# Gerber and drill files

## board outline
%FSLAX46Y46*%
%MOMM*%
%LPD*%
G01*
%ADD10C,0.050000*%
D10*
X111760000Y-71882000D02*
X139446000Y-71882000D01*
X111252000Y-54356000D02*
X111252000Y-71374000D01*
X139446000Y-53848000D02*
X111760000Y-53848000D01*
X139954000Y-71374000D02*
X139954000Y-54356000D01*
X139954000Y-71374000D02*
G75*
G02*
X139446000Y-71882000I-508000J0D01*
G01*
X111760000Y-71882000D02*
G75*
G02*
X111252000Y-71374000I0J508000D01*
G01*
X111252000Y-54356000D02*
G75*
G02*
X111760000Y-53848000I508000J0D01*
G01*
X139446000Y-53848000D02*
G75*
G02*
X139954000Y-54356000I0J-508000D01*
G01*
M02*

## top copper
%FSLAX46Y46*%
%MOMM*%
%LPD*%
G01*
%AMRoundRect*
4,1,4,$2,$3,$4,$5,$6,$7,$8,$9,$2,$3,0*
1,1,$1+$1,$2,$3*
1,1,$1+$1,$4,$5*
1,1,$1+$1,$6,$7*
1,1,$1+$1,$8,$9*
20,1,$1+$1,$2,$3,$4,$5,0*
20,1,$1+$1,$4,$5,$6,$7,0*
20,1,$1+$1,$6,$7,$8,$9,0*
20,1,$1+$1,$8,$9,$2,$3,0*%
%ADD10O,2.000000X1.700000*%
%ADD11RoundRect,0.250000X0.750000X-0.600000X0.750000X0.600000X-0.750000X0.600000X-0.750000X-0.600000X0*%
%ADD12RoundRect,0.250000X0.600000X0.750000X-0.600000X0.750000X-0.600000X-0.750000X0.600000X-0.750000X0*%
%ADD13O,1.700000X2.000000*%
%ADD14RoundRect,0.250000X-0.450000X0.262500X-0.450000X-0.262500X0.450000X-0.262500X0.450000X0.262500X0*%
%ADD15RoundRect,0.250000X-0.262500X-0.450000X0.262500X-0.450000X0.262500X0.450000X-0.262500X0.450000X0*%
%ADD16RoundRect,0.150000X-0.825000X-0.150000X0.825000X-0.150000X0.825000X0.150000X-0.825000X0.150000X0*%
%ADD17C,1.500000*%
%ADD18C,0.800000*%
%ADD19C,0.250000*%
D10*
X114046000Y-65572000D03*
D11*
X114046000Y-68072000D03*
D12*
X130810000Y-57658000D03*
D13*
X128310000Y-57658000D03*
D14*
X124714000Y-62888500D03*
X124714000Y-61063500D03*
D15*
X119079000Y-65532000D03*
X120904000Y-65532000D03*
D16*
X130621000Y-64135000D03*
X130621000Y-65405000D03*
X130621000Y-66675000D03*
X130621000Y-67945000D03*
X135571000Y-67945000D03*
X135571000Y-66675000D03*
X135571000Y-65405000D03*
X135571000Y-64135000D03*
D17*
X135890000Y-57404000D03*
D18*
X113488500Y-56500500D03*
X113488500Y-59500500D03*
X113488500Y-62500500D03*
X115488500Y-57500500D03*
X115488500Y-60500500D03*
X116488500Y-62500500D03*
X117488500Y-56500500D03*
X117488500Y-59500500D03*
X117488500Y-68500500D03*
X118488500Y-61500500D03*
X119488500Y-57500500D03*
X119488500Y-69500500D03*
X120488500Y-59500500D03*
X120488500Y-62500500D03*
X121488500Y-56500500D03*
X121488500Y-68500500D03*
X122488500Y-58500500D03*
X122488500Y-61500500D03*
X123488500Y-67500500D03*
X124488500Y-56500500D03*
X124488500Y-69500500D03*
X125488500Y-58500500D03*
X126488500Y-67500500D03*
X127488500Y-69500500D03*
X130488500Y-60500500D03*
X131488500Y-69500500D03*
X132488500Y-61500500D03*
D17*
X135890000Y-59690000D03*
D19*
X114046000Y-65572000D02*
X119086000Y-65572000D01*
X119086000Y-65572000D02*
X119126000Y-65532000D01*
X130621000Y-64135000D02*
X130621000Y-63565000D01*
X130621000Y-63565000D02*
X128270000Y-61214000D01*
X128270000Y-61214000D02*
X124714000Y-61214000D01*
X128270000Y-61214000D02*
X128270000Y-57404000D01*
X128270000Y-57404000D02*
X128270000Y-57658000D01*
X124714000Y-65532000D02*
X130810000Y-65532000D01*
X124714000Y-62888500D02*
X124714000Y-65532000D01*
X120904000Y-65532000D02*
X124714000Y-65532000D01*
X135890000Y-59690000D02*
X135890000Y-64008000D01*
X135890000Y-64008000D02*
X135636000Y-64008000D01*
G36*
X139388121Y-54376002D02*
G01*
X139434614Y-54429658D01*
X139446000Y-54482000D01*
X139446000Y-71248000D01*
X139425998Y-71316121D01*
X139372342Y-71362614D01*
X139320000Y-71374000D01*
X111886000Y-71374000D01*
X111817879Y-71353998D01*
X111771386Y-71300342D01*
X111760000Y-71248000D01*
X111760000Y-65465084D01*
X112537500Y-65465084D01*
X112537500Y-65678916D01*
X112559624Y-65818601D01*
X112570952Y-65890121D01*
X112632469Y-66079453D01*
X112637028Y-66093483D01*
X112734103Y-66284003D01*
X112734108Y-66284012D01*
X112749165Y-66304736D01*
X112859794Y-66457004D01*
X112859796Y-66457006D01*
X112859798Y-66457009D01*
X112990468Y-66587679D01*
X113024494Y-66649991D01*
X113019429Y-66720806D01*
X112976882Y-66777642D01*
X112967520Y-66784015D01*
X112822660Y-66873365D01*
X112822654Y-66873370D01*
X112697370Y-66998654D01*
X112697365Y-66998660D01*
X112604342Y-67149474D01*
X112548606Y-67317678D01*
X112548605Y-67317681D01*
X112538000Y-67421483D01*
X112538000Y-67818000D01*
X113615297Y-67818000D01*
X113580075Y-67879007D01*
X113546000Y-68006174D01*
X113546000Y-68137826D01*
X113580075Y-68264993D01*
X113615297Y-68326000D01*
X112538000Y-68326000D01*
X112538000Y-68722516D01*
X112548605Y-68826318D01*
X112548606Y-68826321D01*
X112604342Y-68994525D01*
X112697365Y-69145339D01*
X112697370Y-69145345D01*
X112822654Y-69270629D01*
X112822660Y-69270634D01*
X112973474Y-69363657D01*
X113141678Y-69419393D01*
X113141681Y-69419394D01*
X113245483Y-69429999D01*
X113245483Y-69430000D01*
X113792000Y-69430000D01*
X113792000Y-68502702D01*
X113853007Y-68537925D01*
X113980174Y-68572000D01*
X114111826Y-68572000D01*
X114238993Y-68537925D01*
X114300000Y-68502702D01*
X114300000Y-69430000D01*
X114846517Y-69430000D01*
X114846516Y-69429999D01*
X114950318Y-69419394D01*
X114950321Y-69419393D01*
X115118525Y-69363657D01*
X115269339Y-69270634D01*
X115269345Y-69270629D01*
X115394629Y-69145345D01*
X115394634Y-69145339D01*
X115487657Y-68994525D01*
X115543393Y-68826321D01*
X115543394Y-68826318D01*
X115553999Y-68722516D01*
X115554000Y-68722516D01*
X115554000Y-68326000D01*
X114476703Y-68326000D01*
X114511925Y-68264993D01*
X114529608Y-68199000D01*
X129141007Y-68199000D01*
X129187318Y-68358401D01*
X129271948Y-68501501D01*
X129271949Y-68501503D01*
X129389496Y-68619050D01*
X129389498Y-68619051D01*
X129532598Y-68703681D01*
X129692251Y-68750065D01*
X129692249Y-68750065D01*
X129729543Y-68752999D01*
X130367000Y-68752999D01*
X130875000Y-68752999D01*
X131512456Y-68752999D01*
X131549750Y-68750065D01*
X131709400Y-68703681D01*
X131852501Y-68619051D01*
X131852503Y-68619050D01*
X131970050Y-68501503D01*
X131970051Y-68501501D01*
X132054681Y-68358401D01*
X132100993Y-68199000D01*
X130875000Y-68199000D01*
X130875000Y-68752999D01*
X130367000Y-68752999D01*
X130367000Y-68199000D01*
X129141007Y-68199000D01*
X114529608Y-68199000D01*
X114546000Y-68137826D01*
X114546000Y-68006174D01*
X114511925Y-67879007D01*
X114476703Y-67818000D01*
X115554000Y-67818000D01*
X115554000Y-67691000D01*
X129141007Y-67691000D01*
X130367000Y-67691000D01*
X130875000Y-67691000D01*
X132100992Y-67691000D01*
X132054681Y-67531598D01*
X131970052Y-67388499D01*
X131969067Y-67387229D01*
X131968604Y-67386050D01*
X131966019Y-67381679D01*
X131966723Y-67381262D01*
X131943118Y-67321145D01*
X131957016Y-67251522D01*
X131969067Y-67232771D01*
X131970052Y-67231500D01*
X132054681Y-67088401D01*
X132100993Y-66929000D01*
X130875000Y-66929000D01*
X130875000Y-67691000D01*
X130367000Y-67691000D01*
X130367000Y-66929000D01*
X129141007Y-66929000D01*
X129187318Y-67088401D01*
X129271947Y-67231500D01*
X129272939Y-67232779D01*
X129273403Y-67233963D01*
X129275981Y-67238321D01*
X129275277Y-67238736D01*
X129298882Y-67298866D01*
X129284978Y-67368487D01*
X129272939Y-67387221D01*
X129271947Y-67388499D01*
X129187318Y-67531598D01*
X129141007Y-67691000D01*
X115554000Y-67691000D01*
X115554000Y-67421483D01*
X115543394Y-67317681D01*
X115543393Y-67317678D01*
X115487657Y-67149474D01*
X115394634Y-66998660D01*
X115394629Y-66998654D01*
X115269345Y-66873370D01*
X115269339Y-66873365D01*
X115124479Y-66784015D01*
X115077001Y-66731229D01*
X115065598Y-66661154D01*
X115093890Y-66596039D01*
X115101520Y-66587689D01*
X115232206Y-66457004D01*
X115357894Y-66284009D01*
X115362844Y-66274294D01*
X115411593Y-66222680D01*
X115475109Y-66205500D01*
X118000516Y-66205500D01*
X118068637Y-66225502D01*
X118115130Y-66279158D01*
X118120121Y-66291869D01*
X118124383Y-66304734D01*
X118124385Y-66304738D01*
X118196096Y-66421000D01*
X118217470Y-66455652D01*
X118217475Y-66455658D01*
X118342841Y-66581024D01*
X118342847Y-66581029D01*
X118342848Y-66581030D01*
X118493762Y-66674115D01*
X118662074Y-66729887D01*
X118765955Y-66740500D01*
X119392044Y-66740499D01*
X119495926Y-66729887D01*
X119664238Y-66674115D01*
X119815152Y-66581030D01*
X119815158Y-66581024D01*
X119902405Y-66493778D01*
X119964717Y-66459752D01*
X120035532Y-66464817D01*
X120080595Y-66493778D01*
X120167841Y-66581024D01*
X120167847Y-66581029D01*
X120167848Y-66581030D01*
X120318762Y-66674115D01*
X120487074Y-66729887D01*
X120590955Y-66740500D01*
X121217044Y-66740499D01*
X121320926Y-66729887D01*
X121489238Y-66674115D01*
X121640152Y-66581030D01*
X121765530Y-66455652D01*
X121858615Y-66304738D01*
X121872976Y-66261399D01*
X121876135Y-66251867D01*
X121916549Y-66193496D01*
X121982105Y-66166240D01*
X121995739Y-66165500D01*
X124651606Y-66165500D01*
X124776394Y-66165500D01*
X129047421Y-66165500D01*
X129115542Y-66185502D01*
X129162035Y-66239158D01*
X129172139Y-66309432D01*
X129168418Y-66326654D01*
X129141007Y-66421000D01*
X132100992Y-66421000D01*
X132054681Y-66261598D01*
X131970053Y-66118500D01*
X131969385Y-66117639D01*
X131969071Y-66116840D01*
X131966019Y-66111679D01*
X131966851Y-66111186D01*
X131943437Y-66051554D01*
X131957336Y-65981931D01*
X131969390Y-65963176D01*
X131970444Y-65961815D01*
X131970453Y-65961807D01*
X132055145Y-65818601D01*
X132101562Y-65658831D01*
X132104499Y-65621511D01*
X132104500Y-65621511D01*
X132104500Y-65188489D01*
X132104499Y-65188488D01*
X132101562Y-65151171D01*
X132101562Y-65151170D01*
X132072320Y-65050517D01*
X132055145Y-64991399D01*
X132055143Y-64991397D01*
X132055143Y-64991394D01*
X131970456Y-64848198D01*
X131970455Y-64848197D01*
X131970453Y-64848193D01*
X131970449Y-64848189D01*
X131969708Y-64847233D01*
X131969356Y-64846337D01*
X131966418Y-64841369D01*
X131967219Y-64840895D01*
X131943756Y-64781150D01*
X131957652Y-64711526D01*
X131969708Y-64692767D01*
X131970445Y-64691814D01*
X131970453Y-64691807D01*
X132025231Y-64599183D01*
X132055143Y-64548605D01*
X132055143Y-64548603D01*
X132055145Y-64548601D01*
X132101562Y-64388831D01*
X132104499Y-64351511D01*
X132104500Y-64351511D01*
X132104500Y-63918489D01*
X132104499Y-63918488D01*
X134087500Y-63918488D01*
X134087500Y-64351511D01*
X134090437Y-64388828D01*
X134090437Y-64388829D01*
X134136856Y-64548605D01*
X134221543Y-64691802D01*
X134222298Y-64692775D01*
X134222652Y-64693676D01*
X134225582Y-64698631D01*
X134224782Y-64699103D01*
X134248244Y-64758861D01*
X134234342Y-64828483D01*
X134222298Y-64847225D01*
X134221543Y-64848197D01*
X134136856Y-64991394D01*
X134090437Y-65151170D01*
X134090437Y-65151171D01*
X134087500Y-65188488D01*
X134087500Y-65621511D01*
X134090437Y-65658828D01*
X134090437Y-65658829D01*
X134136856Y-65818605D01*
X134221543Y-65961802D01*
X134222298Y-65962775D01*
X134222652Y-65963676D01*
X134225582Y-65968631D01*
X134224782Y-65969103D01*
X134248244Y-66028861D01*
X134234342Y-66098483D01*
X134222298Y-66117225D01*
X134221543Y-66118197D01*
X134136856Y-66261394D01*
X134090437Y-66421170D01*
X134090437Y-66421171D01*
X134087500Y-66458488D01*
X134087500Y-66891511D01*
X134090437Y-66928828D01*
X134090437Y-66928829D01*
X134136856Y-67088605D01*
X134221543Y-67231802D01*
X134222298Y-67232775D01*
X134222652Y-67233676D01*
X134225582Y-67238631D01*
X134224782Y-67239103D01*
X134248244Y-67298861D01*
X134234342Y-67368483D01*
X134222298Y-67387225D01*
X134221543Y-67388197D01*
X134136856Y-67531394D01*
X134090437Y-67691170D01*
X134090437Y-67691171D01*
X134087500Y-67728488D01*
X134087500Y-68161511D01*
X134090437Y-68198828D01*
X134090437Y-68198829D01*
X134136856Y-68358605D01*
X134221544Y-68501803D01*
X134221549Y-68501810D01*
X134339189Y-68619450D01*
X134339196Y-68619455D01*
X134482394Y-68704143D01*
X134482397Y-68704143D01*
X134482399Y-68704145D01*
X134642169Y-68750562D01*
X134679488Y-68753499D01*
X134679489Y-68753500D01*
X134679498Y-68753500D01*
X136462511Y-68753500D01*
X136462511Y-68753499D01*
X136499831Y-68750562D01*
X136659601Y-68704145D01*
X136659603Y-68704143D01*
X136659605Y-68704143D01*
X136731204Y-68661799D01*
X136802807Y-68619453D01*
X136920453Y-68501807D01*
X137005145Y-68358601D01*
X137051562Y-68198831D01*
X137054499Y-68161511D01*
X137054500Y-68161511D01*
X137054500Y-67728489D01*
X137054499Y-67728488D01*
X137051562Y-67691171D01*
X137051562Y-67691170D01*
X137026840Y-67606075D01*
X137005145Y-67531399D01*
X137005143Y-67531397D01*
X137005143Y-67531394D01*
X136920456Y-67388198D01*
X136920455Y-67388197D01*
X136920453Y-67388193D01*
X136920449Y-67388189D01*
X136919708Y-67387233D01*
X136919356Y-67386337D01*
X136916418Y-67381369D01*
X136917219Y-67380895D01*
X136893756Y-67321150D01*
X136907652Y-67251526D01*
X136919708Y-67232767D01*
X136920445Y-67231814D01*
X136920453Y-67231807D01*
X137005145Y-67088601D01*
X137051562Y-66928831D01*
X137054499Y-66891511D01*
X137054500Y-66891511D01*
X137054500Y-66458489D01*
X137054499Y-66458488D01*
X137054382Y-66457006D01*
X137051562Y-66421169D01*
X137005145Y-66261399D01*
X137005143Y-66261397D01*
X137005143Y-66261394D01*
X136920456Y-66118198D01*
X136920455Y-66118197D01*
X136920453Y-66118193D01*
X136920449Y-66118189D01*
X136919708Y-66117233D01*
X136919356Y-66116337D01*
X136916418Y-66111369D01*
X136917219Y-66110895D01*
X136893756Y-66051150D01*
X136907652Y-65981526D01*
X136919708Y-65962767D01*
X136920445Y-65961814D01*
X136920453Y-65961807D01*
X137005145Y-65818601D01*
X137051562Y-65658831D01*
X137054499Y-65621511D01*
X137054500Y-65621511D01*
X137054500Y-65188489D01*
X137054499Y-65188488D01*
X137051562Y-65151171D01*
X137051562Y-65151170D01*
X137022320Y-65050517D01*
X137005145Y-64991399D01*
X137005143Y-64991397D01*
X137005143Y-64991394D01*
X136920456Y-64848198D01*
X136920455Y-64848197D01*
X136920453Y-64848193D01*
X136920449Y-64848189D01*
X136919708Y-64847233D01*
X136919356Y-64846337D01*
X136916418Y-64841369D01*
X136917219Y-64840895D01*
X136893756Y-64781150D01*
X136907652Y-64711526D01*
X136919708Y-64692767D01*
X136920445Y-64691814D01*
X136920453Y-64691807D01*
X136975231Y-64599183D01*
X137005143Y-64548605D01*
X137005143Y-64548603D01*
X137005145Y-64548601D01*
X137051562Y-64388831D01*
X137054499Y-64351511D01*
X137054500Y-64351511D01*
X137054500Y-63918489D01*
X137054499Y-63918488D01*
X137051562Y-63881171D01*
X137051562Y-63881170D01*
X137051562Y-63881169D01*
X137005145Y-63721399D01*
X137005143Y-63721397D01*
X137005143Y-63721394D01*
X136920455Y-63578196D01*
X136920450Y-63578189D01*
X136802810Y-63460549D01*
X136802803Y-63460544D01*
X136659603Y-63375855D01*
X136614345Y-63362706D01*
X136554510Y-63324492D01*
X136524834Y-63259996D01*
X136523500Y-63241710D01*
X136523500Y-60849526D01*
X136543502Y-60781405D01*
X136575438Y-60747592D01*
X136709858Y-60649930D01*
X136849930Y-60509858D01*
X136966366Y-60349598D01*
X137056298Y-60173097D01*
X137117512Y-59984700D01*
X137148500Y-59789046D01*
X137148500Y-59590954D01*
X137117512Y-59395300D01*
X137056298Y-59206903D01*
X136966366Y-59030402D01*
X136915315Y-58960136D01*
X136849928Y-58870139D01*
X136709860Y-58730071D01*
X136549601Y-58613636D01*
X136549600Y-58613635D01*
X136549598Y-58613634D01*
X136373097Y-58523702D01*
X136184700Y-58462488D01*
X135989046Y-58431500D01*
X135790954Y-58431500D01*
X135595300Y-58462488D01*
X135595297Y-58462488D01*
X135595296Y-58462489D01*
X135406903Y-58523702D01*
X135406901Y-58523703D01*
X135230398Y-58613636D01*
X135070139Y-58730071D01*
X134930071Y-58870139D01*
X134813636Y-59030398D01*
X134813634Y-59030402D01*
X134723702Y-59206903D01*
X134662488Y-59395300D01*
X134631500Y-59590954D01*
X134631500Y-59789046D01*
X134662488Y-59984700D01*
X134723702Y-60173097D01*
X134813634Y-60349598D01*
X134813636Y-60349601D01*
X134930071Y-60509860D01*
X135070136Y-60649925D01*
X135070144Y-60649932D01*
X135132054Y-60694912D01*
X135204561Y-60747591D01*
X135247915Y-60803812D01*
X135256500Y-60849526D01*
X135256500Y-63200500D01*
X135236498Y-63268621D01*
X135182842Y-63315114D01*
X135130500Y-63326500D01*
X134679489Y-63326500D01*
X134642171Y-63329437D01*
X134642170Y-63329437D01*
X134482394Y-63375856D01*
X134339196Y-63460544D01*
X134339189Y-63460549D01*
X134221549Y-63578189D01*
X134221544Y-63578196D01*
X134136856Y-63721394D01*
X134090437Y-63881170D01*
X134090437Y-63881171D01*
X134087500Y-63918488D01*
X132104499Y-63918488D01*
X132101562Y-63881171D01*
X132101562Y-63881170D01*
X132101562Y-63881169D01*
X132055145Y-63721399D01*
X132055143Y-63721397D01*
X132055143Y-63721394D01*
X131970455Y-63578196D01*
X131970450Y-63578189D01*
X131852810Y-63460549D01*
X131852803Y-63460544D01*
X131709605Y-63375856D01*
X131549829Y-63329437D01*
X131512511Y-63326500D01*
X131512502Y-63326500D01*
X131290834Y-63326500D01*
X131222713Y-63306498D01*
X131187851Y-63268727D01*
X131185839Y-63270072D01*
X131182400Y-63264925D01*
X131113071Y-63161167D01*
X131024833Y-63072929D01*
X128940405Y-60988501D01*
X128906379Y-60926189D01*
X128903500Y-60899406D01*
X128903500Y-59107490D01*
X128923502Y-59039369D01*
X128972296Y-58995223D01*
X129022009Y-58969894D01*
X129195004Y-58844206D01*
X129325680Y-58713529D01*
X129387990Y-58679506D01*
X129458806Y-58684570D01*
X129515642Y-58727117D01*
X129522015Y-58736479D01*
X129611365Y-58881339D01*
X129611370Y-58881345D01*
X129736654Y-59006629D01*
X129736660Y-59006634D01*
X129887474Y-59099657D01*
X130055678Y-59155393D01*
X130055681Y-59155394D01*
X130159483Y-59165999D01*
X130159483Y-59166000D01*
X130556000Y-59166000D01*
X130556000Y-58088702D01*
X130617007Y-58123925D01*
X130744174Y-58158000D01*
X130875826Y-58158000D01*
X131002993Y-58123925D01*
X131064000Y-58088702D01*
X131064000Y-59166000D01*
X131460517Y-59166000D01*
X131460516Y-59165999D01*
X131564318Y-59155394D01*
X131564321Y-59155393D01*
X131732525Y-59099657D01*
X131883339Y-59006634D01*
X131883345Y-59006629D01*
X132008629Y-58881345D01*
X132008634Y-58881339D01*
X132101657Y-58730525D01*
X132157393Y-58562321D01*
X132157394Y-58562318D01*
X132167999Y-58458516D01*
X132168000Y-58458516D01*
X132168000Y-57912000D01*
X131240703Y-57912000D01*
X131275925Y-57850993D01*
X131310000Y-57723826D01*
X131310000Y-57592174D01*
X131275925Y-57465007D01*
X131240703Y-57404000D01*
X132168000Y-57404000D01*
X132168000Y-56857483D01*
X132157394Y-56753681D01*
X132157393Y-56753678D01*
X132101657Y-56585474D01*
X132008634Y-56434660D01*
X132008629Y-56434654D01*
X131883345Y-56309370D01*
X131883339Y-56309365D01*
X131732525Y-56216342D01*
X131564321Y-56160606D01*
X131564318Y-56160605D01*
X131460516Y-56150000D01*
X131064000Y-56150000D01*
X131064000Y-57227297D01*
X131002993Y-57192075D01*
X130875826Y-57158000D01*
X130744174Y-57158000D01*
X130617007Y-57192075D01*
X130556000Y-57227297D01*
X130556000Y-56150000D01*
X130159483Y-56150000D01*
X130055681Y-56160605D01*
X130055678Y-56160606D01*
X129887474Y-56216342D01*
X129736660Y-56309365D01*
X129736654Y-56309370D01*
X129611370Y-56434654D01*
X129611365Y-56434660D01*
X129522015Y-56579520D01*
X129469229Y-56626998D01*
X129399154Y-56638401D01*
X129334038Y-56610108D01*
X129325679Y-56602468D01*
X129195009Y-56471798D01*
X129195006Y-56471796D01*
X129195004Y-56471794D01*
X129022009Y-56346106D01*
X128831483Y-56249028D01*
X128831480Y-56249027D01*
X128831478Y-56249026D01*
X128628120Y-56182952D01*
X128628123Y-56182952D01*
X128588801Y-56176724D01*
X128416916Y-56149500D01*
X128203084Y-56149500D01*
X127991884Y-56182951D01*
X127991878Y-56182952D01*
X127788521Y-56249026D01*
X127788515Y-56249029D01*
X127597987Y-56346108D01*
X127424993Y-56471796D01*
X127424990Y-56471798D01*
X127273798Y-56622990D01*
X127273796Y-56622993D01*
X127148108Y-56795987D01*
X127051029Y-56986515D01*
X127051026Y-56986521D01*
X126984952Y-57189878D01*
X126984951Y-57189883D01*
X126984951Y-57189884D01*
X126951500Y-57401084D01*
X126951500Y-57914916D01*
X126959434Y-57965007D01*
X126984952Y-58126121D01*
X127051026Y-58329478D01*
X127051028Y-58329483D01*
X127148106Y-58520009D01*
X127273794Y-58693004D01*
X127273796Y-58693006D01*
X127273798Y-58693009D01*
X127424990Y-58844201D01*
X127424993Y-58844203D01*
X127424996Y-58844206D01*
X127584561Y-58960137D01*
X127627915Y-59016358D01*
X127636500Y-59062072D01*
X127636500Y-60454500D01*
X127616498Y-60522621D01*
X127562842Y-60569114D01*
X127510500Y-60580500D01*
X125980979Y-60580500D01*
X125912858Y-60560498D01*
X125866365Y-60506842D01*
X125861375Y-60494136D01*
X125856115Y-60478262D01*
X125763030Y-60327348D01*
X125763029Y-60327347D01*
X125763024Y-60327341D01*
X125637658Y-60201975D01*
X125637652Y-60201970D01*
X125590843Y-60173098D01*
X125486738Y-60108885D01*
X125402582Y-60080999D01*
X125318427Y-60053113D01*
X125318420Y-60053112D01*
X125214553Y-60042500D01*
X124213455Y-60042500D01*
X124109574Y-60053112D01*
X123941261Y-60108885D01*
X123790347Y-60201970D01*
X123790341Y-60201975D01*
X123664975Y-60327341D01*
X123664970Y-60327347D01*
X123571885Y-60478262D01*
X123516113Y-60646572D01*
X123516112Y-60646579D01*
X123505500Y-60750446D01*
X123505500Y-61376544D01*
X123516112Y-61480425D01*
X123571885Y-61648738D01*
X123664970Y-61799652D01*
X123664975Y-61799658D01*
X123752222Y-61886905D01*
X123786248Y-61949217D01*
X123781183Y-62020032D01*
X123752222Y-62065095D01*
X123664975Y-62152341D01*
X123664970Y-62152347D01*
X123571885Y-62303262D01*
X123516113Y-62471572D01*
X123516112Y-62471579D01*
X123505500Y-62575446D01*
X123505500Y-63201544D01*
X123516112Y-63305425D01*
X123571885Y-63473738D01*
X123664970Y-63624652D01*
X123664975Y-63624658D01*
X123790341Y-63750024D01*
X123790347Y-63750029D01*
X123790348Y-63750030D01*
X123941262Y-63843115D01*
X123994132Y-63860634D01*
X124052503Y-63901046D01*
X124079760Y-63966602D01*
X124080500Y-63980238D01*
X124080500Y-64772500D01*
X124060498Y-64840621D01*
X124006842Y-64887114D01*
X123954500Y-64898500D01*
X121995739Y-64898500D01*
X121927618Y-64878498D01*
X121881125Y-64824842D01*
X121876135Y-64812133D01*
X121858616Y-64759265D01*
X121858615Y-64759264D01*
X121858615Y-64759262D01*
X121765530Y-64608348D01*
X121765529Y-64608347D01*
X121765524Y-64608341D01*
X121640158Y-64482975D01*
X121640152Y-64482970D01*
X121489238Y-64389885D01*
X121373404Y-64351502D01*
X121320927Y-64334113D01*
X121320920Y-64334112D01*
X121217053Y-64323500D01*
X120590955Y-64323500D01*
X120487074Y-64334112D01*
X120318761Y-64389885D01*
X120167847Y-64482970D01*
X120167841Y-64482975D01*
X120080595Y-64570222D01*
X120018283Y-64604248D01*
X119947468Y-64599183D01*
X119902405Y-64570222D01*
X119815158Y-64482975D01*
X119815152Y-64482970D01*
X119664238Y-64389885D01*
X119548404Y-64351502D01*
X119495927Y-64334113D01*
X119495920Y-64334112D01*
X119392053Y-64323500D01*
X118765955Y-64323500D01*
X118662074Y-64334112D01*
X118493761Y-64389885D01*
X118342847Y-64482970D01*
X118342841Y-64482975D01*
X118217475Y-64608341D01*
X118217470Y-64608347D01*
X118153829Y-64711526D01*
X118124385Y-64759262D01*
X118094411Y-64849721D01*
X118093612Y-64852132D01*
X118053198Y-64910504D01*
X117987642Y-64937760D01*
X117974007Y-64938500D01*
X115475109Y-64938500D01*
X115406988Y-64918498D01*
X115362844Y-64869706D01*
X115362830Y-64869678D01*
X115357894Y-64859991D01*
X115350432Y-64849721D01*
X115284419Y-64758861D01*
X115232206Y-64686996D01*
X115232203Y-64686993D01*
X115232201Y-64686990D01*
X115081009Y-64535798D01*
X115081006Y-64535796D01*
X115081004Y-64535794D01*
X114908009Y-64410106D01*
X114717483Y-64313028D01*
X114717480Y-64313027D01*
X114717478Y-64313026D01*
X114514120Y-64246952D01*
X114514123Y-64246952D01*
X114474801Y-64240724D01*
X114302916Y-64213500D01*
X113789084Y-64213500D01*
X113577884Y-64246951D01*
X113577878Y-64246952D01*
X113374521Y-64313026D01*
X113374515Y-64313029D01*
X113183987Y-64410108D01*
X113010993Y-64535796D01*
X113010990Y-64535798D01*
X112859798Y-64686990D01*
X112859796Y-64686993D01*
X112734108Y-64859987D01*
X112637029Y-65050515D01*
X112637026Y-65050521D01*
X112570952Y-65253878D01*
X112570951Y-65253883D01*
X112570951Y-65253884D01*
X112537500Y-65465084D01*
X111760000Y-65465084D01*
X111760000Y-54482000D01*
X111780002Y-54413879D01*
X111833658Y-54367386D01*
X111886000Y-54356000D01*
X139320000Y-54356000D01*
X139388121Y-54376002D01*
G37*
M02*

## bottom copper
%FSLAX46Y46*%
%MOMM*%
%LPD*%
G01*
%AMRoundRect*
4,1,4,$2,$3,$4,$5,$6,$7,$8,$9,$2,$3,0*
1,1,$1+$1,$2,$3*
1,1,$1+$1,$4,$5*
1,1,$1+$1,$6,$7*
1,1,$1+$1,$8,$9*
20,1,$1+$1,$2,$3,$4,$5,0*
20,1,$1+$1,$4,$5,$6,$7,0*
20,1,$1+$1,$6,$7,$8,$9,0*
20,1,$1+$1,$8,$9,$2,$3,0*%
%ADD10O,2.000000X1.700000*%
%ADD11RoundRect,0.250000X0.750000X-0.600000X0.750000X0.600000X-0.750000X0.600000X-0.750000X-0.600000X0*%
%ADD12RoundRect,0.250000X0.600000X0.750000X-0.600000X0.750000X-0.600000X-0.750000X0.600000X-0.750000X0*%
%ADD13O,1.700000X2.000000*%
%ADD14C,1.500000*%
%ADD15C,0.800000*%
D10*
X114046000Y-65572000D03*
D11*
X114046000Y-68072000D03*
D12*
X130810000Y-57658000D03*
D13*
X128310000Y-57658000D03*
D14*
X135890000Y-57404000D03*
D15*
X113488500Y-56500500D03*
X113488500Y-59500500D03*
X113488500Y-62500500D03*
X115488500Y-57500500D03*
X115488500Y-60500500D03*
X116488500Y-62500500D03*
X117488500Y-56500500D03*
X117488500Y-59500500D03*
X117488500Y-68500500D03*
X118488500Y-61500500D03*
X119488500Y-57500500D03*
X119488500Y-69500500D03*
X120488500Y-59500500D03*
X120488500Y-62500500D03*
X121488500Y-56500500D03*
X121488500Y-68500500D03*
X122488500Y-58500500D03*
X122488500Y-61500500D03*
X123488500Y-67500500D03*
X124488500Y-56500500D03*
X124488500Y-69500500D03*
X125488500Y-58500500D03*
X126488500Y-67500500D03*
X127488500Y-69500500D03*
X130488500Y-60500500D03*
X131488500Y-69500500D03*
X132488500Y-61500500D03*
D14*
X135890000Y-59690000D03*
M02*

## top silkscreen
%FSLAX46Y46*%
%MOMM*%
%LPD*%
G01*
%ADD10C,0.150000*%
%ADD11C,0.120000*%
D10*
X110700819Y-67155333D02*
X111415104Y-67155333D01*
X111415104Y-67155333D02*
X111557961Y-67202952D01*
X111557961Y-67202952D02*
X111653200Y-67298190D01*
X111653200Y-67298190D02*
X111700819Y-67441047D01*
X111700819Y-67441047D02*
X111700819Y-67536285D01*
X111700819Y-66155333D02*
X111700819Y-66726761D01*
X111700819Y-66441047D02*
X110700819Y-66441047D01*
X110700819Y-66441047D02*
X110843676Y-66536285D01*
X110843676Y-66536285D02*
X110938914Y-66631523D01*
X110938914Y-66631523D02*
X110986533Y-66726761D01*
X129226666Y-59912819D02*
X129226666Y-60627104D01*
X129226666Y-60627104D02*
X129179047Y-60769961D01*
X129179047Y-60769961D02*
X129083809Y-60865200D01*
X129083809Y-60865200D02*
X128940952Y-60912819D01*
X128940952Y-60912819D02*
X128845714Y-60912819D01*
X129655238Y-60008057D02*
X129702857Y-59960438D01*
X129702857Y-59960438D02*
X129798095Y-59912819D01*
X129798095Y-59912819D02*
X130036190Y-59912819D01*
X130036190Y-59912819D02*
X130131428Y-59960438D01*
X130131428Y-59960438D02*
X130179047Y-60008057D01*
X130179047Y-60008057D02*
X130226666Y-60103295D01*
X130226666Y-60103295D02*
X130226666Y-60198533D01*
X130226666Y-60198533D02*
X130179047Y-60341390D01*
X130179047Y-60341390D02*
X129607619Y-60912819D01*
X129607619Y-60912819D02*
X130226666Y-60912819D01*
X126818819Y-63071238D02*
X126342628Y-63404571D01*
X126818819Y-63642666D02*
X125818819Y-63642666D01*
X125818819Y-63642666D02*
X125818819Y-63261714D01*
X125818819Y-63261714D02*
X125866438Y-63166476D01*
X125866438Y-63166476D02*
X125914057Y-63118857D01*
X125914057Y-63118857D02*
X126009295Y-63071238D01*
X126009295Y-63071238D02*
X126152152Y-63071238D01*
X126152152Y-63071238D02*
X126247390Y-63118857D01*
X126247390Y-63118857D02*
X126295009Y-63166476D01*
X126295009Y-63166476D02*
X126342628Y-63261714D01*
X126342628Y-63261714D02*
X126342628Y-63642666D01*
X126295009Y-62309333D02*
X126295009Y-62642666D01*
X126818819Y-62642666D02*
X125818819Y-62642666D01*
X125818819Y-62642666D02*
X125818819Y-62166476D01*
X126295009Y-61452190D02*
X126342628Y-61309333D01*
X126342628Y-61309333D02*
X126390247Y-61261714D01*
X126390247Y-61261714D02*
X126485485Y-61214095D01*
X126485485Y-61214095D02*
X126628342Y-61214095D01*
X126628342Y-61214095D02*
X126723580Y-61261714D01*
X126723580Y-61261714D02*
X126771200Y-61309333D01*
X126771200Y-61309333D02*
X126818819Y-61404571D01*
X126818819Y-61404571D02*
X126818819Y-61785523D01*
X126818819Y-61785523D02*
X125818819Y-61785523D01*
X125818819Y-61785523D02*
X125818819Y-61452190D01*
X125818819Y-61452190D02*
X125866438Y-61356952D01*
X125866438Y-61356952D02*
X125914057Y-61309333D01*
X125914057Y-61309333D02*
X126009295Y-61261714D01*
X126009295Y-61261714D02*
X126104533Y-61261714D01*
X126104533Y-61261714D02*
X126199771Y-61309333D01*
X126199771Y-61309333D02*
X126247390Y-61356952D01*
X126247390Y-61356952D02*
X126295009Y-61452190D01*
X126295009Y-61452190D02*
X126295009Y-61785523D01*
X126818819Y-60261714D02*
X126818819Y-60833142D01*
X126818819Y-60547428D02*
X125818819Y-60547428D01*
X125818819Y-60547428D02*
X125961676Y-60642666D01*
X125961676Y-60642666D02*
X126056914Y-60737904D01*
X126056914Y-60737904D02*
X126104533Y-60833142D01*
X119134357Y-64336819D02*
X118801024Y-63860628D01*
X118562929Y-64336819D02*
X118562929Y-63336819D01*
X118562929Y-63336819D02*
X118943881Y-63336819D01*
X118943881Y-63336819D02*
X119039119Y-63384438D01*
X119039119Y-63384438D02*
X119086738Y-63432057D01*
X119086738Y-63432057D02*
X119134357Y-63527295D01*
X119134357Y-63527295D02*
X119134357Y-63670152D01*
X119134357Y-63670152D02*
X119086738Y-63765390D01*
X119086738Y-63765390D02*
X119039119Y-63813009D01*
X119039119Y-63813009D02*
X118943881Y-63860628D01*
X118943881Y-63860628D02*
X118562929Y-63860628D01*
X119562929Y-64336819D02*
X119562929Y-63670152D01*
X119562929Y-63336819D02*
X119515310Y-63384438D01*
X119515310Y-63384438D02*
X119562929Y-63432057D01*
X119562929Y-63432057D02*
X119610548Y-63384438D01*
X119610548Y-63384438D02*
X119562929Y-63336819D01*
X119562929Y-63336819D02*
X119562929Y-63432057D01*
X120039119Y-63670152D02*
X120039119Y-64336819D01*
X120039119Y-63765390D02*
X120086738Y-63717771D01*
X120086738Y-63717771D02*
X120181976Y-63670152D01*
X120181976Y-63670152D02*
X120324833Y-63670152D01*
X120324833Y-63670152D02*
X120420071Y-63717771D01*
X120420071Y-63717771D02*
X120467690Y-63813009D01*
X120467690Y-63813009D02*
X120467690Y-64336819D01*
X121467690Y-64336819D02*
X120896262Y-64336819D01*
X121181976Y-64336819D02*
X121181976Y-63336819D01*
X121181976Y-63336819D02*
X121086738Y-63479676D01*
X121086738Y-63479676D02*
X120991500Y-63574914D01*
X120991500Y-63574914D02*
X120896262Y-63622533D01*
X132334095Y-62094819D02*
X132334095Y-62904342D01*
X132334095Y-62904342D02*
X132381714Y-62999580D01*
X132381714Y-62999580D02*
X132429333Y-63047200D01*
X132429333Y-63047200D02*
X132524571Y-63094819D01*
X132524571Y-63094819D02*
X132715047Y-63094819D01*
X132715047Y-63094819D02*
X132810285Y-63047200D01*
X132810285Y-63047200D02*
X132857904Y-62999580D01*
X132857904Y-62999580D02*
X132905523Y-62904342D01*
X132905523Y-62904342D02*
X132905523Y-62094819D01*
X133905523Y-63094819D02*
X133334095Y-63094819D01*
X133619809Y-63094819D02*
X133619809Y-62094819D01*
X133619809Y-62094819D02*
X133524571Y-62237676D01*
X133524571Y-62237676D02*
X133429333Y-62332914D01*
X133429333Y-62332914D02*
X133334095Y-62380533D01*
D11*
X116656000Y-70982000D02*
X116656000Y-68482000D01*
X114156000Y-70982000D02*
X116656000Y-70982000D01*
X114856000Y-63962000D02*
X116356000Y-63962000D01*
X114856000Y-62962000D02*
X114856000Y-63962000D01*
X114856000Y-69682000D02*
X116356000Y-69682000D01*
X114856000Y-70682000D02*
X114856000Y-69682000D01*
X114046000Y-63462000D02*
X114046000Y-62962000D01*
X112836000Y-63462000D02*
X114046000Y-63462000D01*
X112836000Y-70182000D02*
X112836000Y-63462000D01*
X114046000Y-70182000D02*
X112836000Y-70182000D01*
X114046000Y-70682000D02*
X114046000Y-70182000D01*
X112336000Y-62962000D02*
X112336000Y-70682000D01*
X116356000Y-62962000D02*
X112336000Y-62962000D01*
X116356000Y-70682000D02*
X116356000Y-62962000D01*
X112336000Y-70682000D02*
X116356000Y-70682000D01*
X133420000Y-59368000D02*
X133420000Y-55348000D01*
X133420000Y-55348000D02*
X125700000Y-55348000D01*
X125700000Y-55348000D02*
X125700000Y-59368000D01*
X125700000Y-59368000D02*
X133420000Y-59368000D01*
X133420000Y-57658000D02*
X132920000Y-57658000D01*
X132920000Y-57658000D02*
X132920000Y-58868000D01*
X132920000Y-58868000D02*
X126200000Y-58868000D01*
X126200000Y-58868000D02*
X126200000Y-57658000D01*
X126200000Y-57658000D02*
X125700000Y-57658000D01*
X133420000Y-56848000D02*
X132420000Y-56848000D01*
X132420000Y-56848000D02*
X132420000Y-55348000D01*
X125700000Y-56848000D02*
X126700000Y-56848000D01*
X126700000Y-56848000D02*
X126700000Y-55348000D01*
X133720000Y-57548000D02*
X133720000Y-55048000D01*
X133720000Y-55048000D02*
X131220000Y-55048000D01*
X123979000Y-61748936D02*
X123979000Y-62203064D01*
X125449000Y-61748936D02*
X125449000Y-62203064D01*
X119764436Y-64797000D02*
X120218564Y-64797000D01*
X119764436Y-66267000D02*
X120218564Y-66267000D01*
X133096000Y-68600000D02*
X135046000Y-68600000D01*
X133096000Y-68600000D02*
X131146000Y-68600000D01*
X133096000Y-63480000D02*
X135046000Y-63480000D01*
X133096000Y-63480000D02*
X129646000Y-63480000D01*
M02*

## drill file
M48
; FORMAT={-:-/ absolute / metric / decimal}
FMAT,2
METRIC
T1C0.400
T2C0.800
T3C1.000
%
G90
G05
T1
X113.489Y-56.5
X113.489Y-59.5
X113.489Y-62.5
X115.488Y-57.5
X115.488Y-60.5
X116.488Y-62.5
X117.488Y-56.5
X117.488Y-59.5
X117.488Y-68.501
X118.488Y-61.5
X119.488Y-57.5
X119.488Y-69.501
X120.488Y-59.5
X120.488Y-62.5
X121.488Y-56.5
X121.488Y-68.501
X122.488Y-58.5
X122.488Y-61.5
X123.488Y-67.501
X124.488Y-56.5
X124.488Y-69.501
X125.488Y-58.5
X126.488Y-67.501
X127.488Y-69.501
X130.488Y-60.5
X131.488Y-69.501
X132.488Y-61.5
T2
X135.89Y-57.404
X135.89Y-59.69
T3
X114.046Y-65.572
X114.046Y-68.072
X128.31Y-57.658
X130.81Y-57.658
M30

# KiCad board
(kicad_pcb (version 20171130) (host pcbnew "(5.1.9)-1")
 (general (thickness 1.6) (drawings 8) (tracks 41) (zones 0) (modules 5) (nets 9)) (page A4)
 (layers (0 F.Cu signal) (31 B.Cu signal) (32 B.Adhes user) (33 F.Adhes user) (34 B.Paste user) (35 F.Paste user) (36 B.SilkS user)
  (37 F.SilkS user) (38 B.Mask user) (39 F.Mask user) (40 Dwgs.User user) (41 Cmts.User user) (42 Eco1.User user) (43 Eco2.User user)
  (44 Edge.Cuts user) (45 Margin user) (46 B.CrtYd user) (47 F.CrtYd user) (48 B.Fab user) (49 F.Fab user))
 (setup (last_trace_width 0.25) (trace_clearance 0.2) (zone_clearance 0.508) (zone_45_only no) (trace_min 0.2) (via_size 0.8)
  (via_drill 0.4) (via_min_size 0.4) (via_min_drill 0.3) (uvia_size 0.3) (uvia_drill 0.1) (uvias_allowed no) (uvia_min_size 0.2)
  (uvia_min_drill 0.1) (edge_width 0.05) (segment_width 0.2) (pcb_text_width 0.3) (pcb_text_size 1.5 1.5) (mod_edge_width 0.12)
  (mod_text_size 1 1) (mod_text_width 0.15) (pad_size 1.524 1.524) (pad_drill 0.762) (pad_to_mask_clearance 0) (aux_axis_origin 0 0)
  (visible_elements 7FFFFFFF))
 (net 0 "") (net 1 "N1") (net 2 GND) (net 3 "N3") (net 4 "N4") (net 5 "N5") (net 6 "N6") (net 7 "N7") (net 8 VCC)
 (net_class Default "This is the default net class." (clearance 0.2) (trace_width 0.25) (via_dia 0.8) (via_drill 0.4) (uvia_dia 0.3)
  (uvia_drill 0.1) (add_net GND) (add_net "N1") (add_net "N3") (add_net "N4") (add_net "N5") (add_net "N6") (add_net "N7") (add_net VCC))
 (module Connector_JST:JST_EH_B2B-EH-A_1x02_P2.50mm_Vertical (layer F.Cu) (at 114.046 68.072 90)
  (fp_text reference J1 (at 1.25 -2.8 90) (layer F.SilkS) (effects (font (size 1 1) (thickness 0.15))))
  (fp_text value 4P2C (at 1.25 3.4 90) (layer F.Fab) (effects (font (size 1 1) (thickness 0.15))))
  (fp_line (start -2.91 2.61) (end -0.41 2.61) (layer F.SilkS) (width 0.12))
  (fp_line (start -2.91 0.11) (end -2.91 2.61) (layer F.SilkS) (width 0.12))
  (fp_line (start 4.11 0.81) (end 4.11 2.31) (layer F.SilkS) (width 0.12))
  (fp_line (start 5.11 0.81) (end 4.11 0.81) (layer F.SilkS) (width 0.12))
  (fp_line (start -1.61 0.81) (end -1.61 2.31) (layer F.SilkS) (width 0.12))
  (fp_line (start -2.61 0.81) (end -1.61 0.81) (layer F.SilkS) (width 0.12))
  (fp_line (start 4.61 0) (end 5.11 0) (layer F.SilkS) (width 0.12))
  (fp_line (start 4.61 -1.21) (end 4.61 0) (layer F.SilkS) (width 0.12))
  (fp_line (start -2.11 -1.21) (end 4.61 -1.21) (layer F.SilkS) (width 0.12))
  (fp_line (start -2.11 0) (end -2.11 -1.21) (layer F.SilkS) (width 0.12))
  (fp_line (start -2.61 0) (end -2.11 0) (layer F.SilkS) (width 0.12))
  (fp_line (start 5.11 -1.71) (end -2.61 -1.71) (layer F.SilkS) (width 0.12))
  (fp_line (start 5.11 2.31) (end 5.11 -1.71) (layer F.SilkS) (width 0.12))
  (fp_line (start -2.61 2.31) (end 5.11 2.31) (layer F.SilkS) (width 0.12))
  (fp_line (start -2.61 -1.71) (end -2.61 2.31) (layer F.SilkS) (width 0.12))
  (pad 2 thru_hole oval (at 2.5 0 90) (size 1.7 2) (drill 1) (layers *.Cu *.Mask) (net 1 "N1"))
  (pad 1 thru_hole roundrect (at 0 0 90) (size 1.7 2) (drill 1) (layers *.Cu *.Mask) (roundrect_rratio 0.147059) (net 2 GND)))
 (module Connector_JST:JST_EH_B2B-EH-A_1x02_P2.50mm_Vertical (layer F.Cu) (at 130.81 57.658 180)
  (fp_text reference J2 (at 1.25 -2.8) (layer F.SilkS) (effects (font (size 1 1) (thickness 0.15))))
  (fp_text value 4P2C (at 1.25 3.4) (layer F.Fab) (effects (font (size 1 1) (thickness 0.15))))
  (fp_line (start -2.61 -1.71) (end -2.61 2.31) (layer F.SilkS) (width 0.12))
  (fp_line (start -2.61 2.31) (end 5.11 2.31) (layer F.SilkS) (width 0.12))
  (fp_line (start 5.11 2.31) (end 5.11 -1.71) (layer F.SilkS) (width 0.12))
  (fp_line (start 5.11 -1.71) (end -2.61 -1.71) (layer F.SilkS) (width 0.12))
  (fp_line (start -2.61 0) (end -2.11 0) (layer F.SilkS) (width 0.12))
  (fp_line (start -2.11 0) (end -2.11 -1.21) (layer F.SilkS) (width 0.12))
  (fp_line (start -2.11 -1.21) (end 4.61 -1.21) (layer F.SilkS) (width 0.12))
  (fp_line (start 4.61 -1.21) (end 4.61 0) (layer F.SilkS) (width 0.12))
  (fp_line (start 4.61 0) (end 5.11 0) (layer F.SilkS) (width 0.12))
  (fp_line (start -2.61 0.81) (end -1.61 0.81) (layer F.SilkS) (width 0.12))
  (fp_line (start -1.61 0.81) (end -1.61 2.31) (layer F.SilkS) (width 0.12))
  (fp_line (start 5.11 0.81) (end 4.11 0.81) (layer F.SilkS) (width 0.12))
  (fp_line (start 4.11 0.81) (end 4.11 2.31) (layer F.SilkS) (width 0.12))
  (fp_line (start -2.91 0.11) (end -2.91 2.61) (layer F.SilkS) (width 0.12))
  (fp_line (start -2.91 2.61) (end -0.41 2.61) (layer F.SilkS) (width 0.12))
  (pad 1 thru_hole roundrect (at 0 0 180) (size 1.7 2) (drill 1) (layers *.Cu *.Mask) (roundrect_rratio 0.147059) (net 2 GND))
  (pad 2 thru_hole oval (at 2.5 0 180) (size 1.7 2) (drill 1) (layers *.Cu *.Mask) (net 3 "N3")))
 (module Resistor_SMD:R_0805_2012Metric (layer F.Cu) (at 124.714 61.976 270)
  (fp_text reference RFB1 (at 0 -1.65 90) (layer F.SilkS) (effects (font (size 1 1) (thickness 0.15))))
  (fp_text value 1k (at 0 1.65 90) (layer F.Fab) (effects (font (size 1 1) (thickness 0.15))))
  (fp_line (start -0.227064 0.735) (end 0.227064 0.735) (layer F.SilkS) (width 0.12))
  (fp_line (start -0.227064 -0.735) (end 0.227064 -0.735) (layer F.SilkS) (width 0.12))
  (pad 2 smd roundrect (at 0.9125 0 270) (size 1.025 1.4) (layers F.Cu F.Paste F.Mask) (roundrect_rratio 0.243902) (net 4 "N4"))
  (pad 1 smd roundrect (at -0.9125 0 270) (size 1.025 1.4) (layers F.Cu F.Paste F.Mask) (roundrect_rratio 0.243902) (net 3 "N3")))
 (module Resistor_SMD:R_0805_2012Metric (layer F.Cu) (at 119.9915 65.532)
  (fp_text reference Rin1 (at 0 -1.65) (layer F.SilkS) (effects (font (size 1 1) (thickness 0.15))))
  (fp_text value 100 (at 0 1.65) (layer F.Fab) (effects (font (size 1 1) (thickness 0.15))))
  (fp_line (start -0.227064 -0.735) (end 0.227064 -0.735) (layer F.SilkS) (width 0.12))
  (fp_line (start -0.227064 0.735) (end 0.227064 0.735) (layer F.SilkS) (width 0.12))
  (pad 1 smd roundrect (at -0.9125 0) (size 1.025 1.4) (layers F.Cu F.Paste F.Mask) (roundrect_rratio 0.243902) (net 1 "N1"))
  (pad 2 smd roundrect (at 0.9125 0) (size 1.025 1.4) (layers F.Cu F.Paste F.Mask) (roundrect_rratio 0.243902) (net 4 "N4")))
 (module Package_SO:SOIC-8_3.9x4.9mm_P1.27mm (layer F.Cu) (at 133.096 66.04)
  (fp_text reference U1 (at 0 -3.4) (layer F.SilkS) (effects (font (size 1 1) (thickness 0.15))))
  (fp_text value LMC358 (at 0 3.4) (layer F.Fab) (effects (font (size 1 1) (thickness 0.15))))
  (fp_line (start 0 2.56) (end 1.95 2.56) (layer F.SilkS) (width 0.12))
  (fp_line (start 0 2.56) (end -1.95 2.56) (layer F.SilkS) (width 0.12))
  (fp_line (start 0 -2.56) (end 1.95 -2.56) (layer F.SilkS) (width 0.12))
  (fp_line (start 0 -2.56) (end -3.45 -2.56) (layer F.SilkS) (width 0.12))
  (pad 1 smd roundrect (at -2.475 -1.905) (size 1.95 0.6) (layers F.Cu F.Paste F.Mask) (roundrect_rratio 0.25) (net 3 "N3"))
  (pad 2 smd roundrect (at -2.475 -0.635) (size 1.95 0.6) (layers F.Cu F.Paste F.Mask) (roundrect_rratio 0.25) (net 4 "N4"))
  (pad 3 smd roundrect (at -2.475 0.635) (size 1.95 0.6) (layers F.Cu F.Paste F.Mask) (roundrect_rratio 0.25) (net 2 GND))
  (pad 4 smd roundrect (at -2.475 1.905) (size 1.95 0.6) (layers F.Cu F.Paste F.Mask) (roundrect_rratio 0.25) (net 2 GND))
  (pad 5 smd roundrect (at 2.475 1.905) (size 1.95 0.6) (layers F.Cu F.Paste F.Mask) (roundrect_rratio 0.25) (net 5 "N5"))
  (pad 6 smd roundrect (at 2.475 0.635) (size 1.95 0.6) (layers F.Cu F.Paste F.Mask) (roundrect_rratio 0.25) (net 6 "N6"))
  (pad 7 smd roundrect (at 2.475 -0.635) (size 1.95 0.6) (layers F.Cu F.Paste F.Mask) (roundrect_rratio 0.25) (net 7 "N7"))
  (pad 8 smd roundrect (at 2.475 -1.905) (size 1.95 0.6) (layers F.Cu F.Paste F.Mask) (roundrect_rratio 0.25) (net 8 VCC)))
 (gr_line (start 111.76 71.882) (end 139.446 71.882) (layer Edge.Cuts) (width 0.05))
 (gr_line (start 111.252 54.356) (end 111.252 71.374) (layer Edge.Cuts) (width 0.05))
 (gr_line (start 139.446 53.848) (end 111.76 53.848) (layer Edge.Cuts) (width 0.05))
 (gr_line (start 139.954 71.374) (end 139.954 54.356) (layer Edge.Cuts) (width 0.05))
 (gr_arc (start 139.446 71.374) (end 139.446 71.882) (angle -90) (layer Edge.Cuts) (width 0.05))
 (gr_arc (start 111.76 71.374) (end 111.252 71.374) (angle -90) (layer Edge.Cuts) (width 0.05))
 (gr_arc (start 111.76 54.356) (end 111.76 53.848) (angle -90) (layer Edge.Cuts) (width 0.05))
 (gr_arc (start 139.446 54.356) (end 139.954 54.356) (angle -90) (layer Edge.Cuts) (width 0.05))
 (segment (start 114.046 65.572) (end 119.086 65.572) (width 0.25) (layer F.Cu) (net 1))
 (segment (start 119.086 65.572) (end 119.126 65.532) (width 0.25) (layer F.Cu) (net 1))
 (via (at 135.89 57.404) (size 1.5) (drill 0.8) (layers F.Cu B.Cu) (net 2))
 (via (at 113.4885 56.5005) (size 0.8) (drill 0.4) (layers F.Cu B.Cu) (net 2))
 (via (at 113.4885 59.5005) (size 0.8) (drill 0.4) (layers F.Cu B.Cu) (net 2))
 (via (at 113.4885 62.5005) (size 0.8) (drill 0.4) (layers F.Cu B.Cu) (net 2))
 (via (at 115.4885 57.5005) (size 0.8) (drill 0.4) (layers F.Cu B.Cu) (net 2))
 (via (at 115.4885 60.5005) (size 0.8) (drill 0.4) (layers F.Cu B.Cu) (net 2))
 (via (at 116.4885 62.5005) (size 0.8) (drill 0.4) (layers F.Cu B.Cu) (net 2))
 (via (at 117.4885 56.5005) (size 0.8) (drill 0.4) (layers F.Cu B.Cu) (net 2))
 (via (at 117.4885 59.5005) (size 0.8) (drill 0.4) (layers F.Cu B.Cu) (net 2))
 (via (at 117.4885 68.5005) (size 0.8) (drill 0.4) (layers F.Cu B.Cu) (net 2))
 (via (at 118.4885 61.5005) (size 0.8) (drill 0.4) (layers F.Cu B.Cu) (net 2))
 (via (at 119.4885 57.5005) (size 0.8) (drill 0.4) (layers F.Cu B.Cu) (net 2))
 (via (at 119.4885 69.5005) (size 0.8) (drill 0.4) (layers F.Cu B.Cu) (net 2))
 (via (at 120.4885 59.5005) (size 0.8) (drill 0.4) (layers F.Cu B.Cu) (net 2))
 (via (at 120.4885 62.5005) (size 0.8) (drill 0.4) (layers F.Cu B.Cu) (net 2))
 (via (at 121.4885 56.5005) (size 0.8) (drill 0.4) (layers F.Cu B.Cu) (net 2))
 (via (at 121.4885 68.5005) (size 0.8) (drill 0.4) (layers F.Cu B.Cu) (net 2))
 (via (at 122.4885 58.5005) (size 0.8) (drill 0.4) (layers F.Cu B.Cu) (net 2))
 (via (at 122.4885 61.5005) (size 0.8) (drill 0.4) (layers F.Cu B.Cu) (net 2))
 (via (at 123.4885 67.5005) (size 0.8) (drill 0.4) (layers F.Cu B.Cu) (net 2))
 (via (at 124.4885 56.5005) (size 0.8) (drill 0.4) (layers F.Cu B.Cu) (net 2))
 (via (at 124.4885 69.5005) (size 0.8) (drill 0.4) (layers F.Cu B.Cu) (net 2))
 (via (at 125.4885 58.5005) (size 0.8) (drill 0.4) (layers F.Cu B.Cu) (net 2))
 (via (at 126.4885 67.5005) (size 0.8) (drill 0.4) (layers F.Cu B.Cu) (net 2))
 (via (at 127.4885 69.5005) (size 0.8) (drill 0.4) (layers F.Cu B.Cu) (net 2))
 (via (at 130.4885 60.5005) (size 0.8) (drill 0.4) (layers F.Cu B.Cu) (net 2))
 (via (at 131.4885 69.5005) (size 0.8) (drill 0.4) (layers F.Cu B.Cu) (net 2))
 (via (at 132.4885 61.5005) (size 0.8) (drill 0.4) (layers F.Cu B.Cu) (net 2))
 (segment (start 130.621 64.135) (end 130.621 63.565) (width 0.25) (layer F.Cu) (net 3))
 (segment (start 130.621 63.565) (end 128.27 61.214) (width 0.25) (layer F.Cu) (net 3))
 (segment (start 128.27 61.214) (end 124.714 61.214) (width 0.25) (layer F.Cu) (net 3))
 (segment (start 128.27 61.214) (end 128.27 57.404) (width 0.25) (layer F.Cu) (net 3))
 (segment (start 128.27 57.404) (end 128.27 57.658) (width 0.25) (layer F.Cu) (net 3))
 (segment (start 124.714 65.532) (end 130.81 65.532) (width 0.25) (layer F.Cu) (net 4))
 (segment (start 124.714 62.8885) (end 124.714 65.532) (width 0.25) (layer F.Cu) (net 4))
 (segment (start 120.904 65.532) (end 124.714 65.532) (width 0.25) (layer F.Cu) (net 4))
 (via (at 135.89 59.69) (size 1.5) (drill 0.8) (layers F.Cu B.Cu) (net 8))
 (segment (start 135.89 59.69) (end 135.89 64.008) (width 0.25) (layer F.Cu) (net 8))
 (segment (start 135.89 64.008) (end 135.636 64.008) (width 0.25) (layer F.Cu) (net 8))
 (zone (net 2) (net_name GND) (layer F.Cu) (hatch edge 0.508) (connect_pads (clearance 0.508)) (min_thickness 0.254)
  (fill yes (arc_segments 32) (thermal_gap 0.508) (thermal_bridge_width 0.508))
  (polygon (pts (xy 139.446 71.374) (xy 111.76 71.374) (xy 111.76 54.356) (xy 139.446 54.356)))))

